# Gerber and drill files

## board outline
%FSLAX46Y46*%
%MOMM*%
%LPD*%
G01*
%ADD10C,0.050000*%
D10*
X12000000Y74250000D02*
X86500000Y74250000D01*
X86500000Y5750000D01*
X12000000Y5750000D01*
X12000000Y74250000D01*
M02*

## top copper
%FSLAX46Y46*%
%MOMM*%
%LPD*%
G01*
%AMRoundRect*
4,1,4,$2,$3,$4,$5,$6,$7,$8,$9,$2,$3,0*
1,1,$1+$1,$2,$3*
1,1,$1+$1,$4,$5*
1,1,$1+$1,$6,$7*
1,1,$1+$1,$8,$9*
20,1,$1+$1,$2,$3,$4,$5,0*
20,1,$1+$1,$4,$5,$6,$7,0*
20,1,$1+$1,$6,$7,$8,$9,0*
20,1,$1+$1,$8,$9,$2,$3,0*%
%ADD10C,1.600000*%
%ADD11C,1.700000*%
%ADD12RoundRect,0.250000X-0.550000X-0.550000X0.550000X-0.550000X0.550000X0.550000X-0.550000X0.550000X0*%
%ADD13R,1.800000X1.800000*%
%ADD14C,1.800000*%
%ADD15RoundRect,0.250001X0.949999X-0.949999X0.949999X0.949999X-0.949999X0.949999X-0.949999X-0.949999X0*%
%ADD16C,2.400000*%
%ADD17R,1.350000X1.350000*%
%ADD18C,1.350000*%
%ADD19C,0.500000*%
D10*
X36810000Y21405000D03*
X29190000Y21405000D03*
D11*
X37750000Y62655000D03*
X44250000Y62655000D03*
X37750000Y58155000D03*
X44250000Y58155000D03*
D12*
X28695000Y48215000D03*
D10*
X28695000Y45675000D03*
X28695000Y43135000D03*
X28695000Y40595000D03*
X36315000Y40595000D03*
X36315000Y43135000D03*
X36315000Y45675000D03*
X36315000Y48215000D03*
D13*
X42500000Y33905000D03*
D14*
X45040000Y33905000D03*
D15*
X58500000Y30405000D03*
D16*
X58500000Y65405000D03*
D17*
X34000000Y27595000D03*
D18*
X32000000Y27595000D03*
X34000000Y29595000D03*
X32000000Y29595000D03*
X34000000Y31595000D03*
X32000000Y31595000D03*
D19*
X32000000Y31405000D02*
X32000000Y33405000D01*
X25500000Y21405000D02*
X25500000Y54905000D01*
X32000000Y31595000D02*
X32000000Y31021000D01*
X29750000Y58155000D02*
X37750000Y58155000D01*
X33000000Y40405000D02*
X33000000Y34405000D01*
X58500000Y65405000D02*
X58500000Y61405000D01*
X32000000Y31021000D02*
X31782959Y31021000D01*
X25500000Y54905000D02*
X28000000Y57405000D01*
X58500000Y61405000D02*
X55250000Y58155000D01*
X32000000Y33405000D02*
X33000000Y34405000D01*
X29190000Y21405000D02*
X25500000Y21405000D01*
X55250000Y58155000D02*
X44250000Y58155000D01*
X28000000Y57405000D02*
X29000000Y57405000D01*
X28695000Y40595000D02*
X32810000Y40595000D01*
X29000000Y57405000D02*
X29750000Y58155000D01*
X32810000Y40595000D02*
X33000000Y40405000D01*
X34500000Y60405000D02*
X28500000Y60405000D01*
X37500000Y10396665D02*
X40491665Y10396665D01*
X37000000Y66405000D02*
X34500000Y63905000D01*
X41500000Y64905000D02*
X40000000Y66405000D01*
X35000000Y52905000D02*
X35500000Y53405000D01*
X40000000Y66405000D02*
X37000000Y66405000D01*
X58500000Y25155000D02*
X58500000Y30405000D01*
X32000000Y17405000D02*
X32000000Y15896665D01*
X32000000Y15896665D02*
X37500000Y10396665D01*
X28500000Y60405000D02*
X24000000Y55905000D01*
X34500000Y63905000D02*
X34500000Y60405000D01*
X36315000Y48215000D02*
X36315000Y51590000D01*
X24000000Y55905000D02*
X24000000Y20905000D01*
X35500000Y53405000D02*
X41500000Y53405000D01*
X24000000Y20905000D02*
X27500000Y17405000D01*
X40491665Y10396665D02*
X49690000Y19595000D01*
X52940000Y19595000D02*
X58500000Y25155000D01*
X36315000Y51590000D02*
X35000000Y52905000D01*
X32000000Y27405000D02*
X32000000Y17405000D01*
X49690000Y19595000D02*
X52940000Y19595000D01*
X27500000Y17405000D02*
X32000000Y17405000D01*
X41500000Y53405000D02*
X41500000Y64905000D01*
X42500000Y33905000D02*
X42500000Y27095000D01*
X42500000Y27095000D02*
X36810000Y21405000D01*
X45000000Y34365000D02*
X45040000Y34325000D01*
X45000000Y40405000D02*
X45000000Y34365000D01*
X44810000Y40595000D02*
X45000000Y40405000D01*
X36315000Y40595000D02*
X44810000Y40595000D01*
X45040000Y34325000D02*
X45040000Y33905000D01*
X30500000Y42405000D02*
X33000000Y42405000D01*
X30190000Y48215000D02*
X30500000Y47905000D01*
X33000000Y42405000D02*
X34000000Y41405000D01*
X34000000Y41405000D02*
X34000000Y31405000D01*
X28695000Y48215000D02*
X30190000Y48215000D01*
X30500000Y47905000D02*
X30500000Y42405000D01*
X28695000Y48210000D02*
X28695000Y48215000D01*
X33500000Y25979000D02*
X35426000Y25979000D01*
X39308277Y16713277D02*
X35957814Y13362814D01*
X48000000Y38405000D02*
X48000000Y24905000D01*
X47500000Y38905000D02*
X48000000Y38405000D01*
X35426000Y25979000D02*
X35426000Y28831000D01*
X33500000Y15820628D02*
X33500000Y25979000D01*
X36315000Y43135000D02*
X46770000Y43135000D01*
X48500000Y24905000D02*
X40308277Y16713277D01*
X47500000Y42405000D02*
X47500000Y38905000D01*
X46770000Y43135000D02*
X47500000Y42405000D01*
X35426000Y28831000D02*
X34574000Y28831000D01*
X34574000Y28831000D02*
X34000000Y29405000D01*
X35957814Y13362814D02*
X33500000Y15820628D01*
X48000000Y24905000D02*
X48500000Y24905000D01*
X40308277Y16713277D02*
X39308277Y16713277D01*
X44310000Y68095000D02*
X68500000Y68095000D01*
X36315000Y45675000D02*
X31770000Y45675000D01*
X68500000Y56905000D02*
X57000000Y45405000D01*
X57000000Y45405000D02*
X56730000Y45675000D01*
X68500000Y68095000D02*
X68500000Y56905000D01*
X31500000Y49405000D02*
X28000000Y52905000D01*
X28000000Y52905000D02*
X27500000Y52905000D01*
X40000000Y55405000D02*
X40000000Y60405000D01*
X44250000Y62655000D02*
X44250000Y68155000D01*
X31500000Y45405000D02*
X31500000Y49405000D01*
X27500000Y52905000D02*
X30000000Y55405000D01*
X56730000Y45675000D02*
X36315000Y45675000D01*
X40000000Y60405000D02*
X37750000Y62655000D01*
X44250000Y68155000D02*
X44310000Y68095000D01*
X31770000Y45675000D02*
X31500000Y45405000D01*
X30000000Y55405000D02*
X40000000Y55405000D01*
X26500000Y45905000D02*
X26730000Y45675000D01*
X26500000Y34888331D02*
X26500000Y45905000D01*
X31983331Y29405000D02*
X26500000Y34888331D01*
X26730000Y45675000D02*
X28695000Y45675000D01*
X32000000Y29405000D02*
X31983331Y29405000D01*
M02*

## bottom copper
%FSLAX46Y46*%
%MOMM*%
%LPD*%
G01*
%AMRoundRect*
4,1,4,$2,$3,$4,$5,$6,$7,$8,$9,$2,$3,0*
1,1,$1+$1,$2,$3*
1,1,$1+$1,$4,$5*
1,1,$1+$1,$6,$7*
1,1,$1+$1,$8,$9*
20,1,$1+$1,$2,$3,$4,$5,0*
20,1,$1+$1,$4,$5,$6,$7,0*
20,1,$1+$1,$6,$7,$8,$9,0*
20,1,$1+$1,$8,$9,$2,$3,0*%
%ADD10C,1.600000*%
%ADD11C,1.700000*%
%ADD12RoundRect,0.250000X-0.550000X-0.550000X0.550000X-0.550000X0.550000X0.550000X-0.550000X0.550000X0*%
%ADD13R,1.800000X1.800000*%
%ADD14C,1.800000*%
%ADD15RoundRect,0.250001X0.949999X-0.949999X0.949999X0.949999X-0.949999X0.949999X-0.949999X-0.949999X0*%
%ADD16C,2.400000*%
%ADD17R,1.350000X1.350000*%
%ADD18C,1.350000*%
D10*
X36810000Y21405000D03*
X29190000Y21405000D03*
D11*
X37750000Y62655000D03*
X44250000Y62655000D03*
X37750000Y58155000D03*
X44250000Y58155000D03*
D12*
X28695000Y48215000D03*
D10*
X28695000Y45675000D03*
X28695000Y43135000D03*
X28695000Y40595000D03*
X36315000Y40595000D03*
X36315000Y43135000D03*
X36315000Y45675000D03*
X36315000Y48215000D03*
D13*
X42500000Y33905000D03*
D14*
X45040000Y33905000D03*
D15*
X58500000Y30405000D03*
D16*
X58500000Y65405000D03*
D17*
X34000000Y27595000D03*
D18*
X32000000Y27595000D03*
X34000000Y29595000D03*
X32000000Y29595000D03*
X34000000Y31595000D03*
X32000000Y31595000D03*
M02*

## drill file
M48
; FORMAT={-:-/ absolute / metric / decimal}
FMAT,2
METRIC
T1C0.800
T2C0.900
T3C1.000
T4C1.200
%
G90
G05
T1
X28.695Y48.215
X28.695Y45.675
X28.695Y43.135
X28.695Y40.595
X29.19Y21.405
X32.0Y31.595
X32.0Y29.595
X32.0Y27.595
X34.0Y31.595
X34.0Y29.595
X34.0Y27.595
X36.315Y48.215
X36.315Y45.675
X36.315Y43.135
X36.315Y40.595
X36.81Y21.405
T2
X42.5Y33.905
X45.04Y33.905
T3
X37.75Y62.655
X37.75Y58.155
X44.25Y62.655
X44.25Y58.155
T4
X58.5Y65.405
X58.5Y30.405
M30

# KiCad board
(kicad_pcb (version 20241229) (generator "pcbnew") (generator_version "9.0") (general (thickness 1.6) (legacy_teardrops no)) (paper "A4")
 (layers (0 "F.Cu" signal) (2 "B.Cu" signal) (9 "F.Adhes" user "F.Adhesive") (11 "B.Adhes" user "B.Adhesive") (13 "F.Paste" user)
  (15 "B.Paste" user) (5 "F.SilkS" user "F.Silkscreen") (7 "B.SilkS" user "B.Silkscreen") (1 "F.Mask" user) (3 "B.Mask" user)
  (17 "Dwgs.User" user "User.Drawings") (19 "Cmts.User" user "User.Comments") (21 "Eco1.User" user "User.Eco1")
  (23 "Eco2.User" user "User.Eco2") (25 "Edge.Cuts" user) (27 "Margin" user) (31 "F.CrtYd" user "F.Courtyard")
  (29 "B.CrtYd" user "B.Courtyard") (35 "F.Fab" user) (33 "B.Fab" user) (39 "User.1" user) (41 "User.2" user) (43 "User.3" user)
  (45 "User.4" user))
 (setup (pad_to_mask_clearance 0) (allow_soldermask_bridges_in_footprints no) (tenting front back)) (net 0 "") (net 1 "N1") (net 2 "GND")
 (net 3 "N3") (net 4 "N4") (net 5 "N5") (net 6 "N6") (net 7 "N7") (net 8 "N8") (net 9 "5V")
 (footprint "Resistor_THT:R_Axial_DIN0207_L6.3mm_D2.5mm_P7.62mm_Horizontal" (layer "F.Cu") (at 36.81 -21.405 180)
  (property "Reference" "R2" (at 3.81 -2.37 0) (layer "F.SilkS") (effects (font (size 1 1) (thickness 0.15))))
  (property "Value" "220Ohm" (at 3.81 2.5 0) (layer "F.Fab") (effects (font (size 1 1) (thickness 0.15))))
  (pad "1" thru_hole circle (at 0 0 180) (size 1.6 1.6) (drill 0.8) (layers "*.Cu" "*.Mask") (remove_unused_layers no) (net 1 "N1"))
  (pad "2" thru_hole circle (at 7.62 0 180) (size 1.6 1.6) (drill 0.8) (layers "*.Cu" "*.Mask") (remove_unused_layers no) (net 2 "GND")))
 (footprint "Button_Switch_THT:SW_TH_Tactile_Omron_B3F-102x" (layer "F.Cu") (at 37.75 -62.655)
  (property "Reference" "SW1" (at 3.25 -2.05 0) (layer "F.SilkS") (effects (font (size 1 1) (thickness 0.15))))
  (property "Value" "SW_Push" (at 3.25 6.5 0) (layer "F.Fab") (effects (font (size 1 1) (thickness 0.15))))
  (pad "1" thru_hole circle (at 0 0) (size 1.7 1.7) (drill 1) (layers "*.Cu" "*.Mask") (remove_unused_layers no) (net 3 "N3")
   (thermal_bridge_angle 90))
  (pad "1" thru_hole circle (at 6.5 0) (size 1.7 1.7) (drill 1) (layers "*.Cu" "*.Mask") (remove_unused_layers no) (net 3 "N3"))
  (pad "2" thru_hole circle (at 0 4.5) (size 1.7 1.7) (drill 1) (layers "*.Cu" "*.Mask") (remove_unused_layers no) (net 2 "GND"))
  (pad "2" thru_hole circle (at 6.5 4.5) (size 1.7 1.7) (drill 1) (layers "*.Cu" "*.Mask") (remove_unused_layers no) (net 2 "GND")))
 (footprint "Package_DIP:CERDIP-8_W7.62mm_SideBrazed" (layer "F.Cu") (at 28.695 -48.215)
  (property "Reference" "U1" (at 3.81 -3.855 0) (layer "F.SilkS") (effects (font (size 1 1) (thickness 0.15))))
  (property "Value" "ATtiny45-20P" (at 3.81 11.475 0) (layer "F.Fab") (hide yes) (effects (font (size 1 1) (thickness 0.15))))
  (pad "1" thru_hole roundrect (at 0 0) (size 1.6 1.6) (drill 0.8) (layers "*.Cu" "*.Mask") (remove_unused_layers no)
   (roundrect_rratio 0.15625) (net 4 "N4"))
  (pad "2" thru_hole circle (at 0 2.54) (size 1.6 1.6) (drill 0.8) (layers "*.Cu" "*.Mask") (remove_unused_layers no) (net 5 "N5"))
  (pad "3" thru_hole circle (at 0 5.08) (size 1.6 1.6) (drill 0.8) (layers "*.Cu" "*.Mask") (remove_unused_layers no) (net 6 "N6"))
  (pad "4" thru_hole circle (at 0 7.62) (size 1.6 1.6) (drill 0.8) (layers "*.Cu" "*.Mask") (remove_unused_layers no) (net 2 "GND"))
  (pad "5" thru_hole circle (at 7.62 7.62) (size 1.6 1.6) (drill 0.8) (layers "*.Cu" "*.Mask") (remove_unused_layers no) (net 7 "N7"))
  (pad "6" thru_hole circle (at 7.62 5.08) (size 1.6 1.6) (drill 0.8) (layers "*.Cu" "*.Mask") (remove_unused_layers no) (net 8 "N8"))
  (pad "7" thru_hole circle (at 7.62 2.54) (size 1.6 1.6) (drill 0.8) (layers "*.Cu" "*.Mask") (remove_unused_layers no) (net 3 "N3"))
  (pad "8" thru_hole circle (at 7.62 0) (size 1.6 1.6) (drill 0.8) (layers "*.Cu" "*.Mask") (remove_unused_layers no) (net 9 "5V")))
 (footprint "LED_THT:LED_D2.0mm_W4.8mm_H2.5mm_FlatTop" (layer "F.Cu") (at 42.5 -33.905)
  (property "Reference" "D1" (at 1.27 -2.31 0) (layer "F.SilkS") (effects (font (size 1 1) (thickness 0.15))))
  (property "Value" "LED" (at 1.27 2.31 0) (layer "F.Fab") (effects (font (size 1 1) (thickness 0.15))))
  (pad "1" thru_hole rect (at 0 0) (size 1.8 1.8) (drill 0.9) (layers "*.Cu" "*.Mask") (remove_unused_layers no) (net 1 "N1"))
  (pad "2" thru_hole circle (at 2.54 0) (size 1.8 1.8) (drill 0.9) (layers "*.Cu" "*.Mask") (remove_unused_layers no) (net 7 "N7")))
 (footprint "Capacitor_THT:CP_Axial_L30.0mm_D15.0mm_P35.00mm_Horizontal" (layer "F.Cu") (at 58.5 -30.405 90)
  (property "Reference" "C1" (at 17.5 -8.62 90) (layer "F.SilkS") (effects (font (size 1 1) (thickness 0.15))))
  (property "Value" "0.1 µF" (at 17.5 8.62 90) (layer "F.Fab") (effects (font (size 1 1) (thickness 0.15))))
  (pad "1" thru_hole roundrect (at 0 0 90) (size 2.4 2.4) (drill 1.2) (layers "*.Cu" "*.Mask") (remove_unused_layers no)
   (roundrect_rratio 0.104167) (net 9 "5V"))
  (pad "2" thru_hole circle (at 35 0 90) (size 2.4 2.4) (drill 1.2) (layers "*.Cu" "*.Mask") (remove_unused_layers no) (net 2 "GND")))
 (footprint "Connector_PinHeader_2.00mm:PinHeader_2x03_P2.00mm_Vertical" (layer "F.Cu") (at 34 -27.595 180)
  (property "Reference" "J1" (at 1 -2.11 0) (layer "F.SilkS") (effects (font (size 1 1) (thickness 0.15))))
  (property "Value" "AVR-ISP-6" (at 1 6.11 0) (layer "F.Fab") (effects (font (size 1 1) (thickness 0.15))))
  (pad "0" thru_hole rect (at 0 0 180) (size 1.35 1.35) (drill 0.8) (layers "*.Cu" "*.Mask") (remove_unused_layers no) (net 6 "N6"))
  (pad "2" thru_hole circle (at 2 0 180) (size 1.35 1.35) (drill 0.8) (layers "*.Cu" "*.Mask") (remove_unused_layers no) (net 9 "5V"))
  (pad "3" thru_hole circle (at 0 2 180) (size 1.35 1.35) (drill 0.8) (layers "*.Cu" "*.Mask") (remove_unused_layers no) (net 8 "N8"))
  (pad "4" thru_hole circle (at 2 2 180) (size 1.35 1.35) (drill 0.8) (layers "*.Cu" "*.Mask") (remove_unused_layers no) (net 5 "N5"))
  (pad "5" thru_hole circle (at 0 4 180) (size 1.35 1.35) (drill 0.8) (layers "*.Cu" "*.Mask") (remove_unused_layers no) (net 4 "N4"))
  (pad "6" thru_hole circle (at 2 4 180) (size 1.35 1.35) (drill 0.8) (layers "*.Cu" "*.Mask") (remove_unused_layers no) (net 2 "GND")))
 (gr_rect (start 12 -74.25) (end 86.5 -5.75) (stroke (width 0.05) (type default)) (fill no) (layer "Edge.Cuts"))
 (segment (start 32 -31.405) (end 32 -33.405) (width 0.5) (layer "F.Cu") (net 2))
 (segment (start 25.5 -21.405) (end 25.5 -54.905) (width 0.5) (layer "F.Cu") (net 2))
 (segment (start 32 -31.595) (end 32 -31.021) (width 0.5) (layer "F.Cu") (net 2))
 (segment (start 29.75 -58.155) (end 37.75 -58.155) (width 0.5) (layer "F.Cu") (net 2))
 (segment (start 33 -40.405) (end 33 -34.405) (width 0.5) (layer "F.Cu") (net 2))
 (segment (start 58.5 -65.405) (end 58.5 -61.405) (width 0.5) (layer "F.Cu") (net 2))
 (segment (start 32 -31.021) (end 31.782959 -31.021) (width 0.5) (layer "F.Cu") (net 2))
 (segment (start 25.5 -54.905) (end 28 -57.405) (width 0.5) (layer "F.Cu") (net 2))
 (segment (start 58.5 -61.405) (end 55.25 -58.155) (width 0.5) (layer "F.Cu") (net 2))
 (segment (start 32 -33.405) (end 33 -34.405) (width 0.5) (layer "F.Cu") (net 2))
 (segment (start 29.19 -21.405) (end 25.5 -21.405) (width 0.5) (layer "F.Cu") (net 2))
 (segment (start 55.25 -58.155) (end 44.25 -58.155) (width 0.5) (layer "F.Cu") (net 2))
 (segment (start 28 -57.405) (end 29 -57.405) (width 0.5) (layer "F.Cu") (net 2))
 (segment (start 28.695 -40.595) (end 32.81 -40.595) (width 0.5) (layer "F.Cu") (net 2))
 (segment (start 29 -57.405) (end 29.75 -58.155) (width 0.5) (layer "F.Cu") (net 2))
 (segment (start 32.81 -40.595) (end 33 -40.405) (width 0.5) (layer "F.Cu") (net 2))
 (segment (start 34.5 -60.405) (end 28.5 -60.405) (width 0.5) (layer "F.Cu") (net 9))
 (segment (start 37.5 -10.396665) (end 40.491665 -10.396665) (width 0.5) (layer "F.Cu") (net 9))
 (segment (start 37 -66.405) (end 34.5 -63.905) (width 0.5) (layer "F.Cu") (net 9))
 (segment (start 41.5 -64.905) (end 40 -66.405) (width 0.5) (layer "F.Cu") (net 9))
 (segment (start 35 -52.905) (end 35.5 -53.405) (width 0.5) (layer "F.Cu") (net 9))
 (segment (start 40 -66.405) (end 37 -66.405) (width 0.5) (layer "F.Cu") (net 9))
 (segment (start 58.5 -25.155) (end 58.5 -30.405) (width 0.5) (layer "F.Cu") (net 9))
 (segment (start 32 -17.405) (end 32 -15.896665) (width 0.5) (layer "F.Cu") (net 9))
 (segment (start 32 -15.896665) (end 37.5 -10.396665) (width 0.5) (layer "F.Cu") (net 9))
 (segment (start 28.5 -60.405) (end 24 -55.905) (width 0.5) (layer "F.Cu") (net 9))
 (segment (start 34.5 -63.905) (end 34.5 -60.405) (width 0.5) (layer "F.Cu") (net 9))
 (segment (start 36.315 -48.215) (end 36.315 -51.59) (width 0.5) (layer "F.Cu") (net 9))
 (segment (start 24 -55.905) (end 24 -20.905) (width 0.5) (layer "F.Cu") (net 9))
 (segment (start 35.5 -53.405) (end 41.5 -53.405) (width 0.5) (layer "F.Cu") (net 9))
 (segment (start 24 -20.905) (end 27.5 -17.405) (width 0.5) (layer "F.Cu") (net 9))
 (segment (start 40.491665 -10.396665) (end 49.69 -19.595) (width 0.5) (layer "F.Cu") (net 9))
 (segment (start 52.94 -19.595) (end 58.5 -25.155) (width 0.5) (layer "F.Cu") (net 9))
 (segment (start 36.315 -51.59) (end 35 -52.905) (width 0.5) (layer "F.Cu") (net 9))
 (segment (start 32 -27.405) (end 32 -17.405) (width 0.5) (layer "F.Cu") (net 9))
 (segment (start 49.69 -19.595) (end 52.94 -19.595) (width 0.5) (layer "F.Cu") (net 9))
 (segment (start 27.5 -17.405) (end 32 -17.405) (width 0.5) (layer "F.Cu") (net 9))
 (segment (start 41.5 -53.405) (end 41.5 -64.905) (width 0.5) (layer "F.Cu") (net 9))
 (segment (start 42.5 -33.905) (end 42.5 -27.095) (width 0.5) (layer "F.Cu") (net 1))
 (segment (start 42.5 -27.095) (end 36.81 -21.405) (width 0.5) (layer "F.Cu") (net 1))
 (segment (start 45 -34.365) (end 45.04 -34.325) (width 0.5) (layer "F.Cu") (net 7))
 (segment (start 45 -40.405) (end 45 -34.365) (width 0.5) (layer "F.Cu") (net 7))
 (segment (start 44.81 -40.595) (end 45 -40.405) (width 0.5) (layer "F.Cu") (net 7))
 (segment (start 36.315 -40.595) (end 44.81 -40.595) (width 0.5) (layer "F.Cu") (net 7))
 (segment (start 45.04 -34.325) (end 45.04 -33.905) (width 0.5) (layer "F.Cu") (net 7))
 (segment (start 30.5 -42.405) (end 33 -42.405) (width 0.5) (layer "F.Cu") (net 4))
 (segment (start 30.19 -48.215) (end 30.5 -47.905) (width 0.5) (layer "F.Cu") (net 4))
 (segment (start 33 -42.405) (end 34 -41.405) (width 0.5) (layer "F.Cu") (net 4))
 (segment (start 34 -41.405) (end 34 -31.405) (width 0.5) (layer "F.Cu") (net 4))
 (segment (start 28.695 -48.215) (end 30.19 -48.215) (width 0.5) (layer "F.Cu") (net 4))
 (segment (start 30.5 -47.905) (end 30.5 -42.405) (width 0.5) (layer "F.Cu") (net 4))
 (segment (start 28.695 -48.21) (end 28.695 -48.215) (width 0.5) (layer "F.Cu") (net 4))
 (segment (start 33.5 -25.979) (end 35.426 -25.979) (width 0.5) (layer "F.Cu") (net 8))
 (segment (start 39.308277 -16.713277) (end 35.957814 -13.362814) (width 0.5) (layer "F.Cu") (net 8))
 (segment (start 48 -38.405) (end 48 -24.905) (width 0.5) (layer "F.Cu") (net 8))
 (segment (start 47.5 -38.905) (end 48 -38.405) (width 0.5) (layer "F.Cu") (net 8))
 (segment (start 35.426 -25.979) (end 35.426 -28.831) (width 0.5) (layer "F.Cu") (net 8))
 (segment (start 33.5 -15.820628) (end 33.5 -25.979) (width 0.5) (layer "F.Cu") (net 8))
 (segment (start 36.315 -43.135) (end 46.77 -43.135) (width 0.5) (layer "F.Cu") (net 8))
 (segment (start 48.5 -24.905) (end 40.308277 -16.713277) (width 0.5) (layer "F.Cu") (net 8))
 (segment (start 47.5 -42.405) (end 47.5 -38.905) (width 0.5) (layer "F.Cu") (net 8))
 (segment (start 46.77 -43.135) (end 47.5 -42.405) (width 0.5) (layer "F.Cu") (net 8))
 (segment (start 35.426 -28.831) (end 34.574 -28.831) (width 0.5) (layer "F.Cu") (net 8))
 (segment (start 34.574 -28.831) (end 34 -29.405) (width 0.5) (layer "F.Cu") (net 8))
 (segment (start 35.957814 -13.362814) (end 33.5 -15.820628) (width 0.5) (layer "F.Cu") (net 8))
 (segment (start 48 -24.905) (end 48.5 -24.905) (width 0.5) (layer "F.Cu") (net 8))
 (segment (start 40.308277 -16.713277) (end 39.308277 -16.713277) (width 0.5) (layer "F.Cu") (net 8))
 (segment (start 44.31 -68.095) (end 68.5 -68.095) (width 0.5) (layer "F.Cu") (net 3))
 (segment (start 36.315 -45.675) (end 31.77 -45.675) (width 0.5) (layer "F.Cu") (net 3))
 (segment (start 68.5 -56.905) (end 57 -45.405) (width 0.5) (layer "F.Cu") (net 3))
 (segment (start 57 -45.405) (end 56.73 -45.675) (width 0.5) (layer "F.Cu") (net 3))
 (segment (start 68.5 -68.095) (end 68.5 -56.905) (width 0.5) (layer "F.Cu") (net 3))
 (segment (start 31.5 -49.405) (end 28 -52.905) (width 0.5) (layer "F.Cu") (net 3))
 (segment (start 28 -52.905) (end 27.5 -52.905) (width 0.5) (layer "F.Cu") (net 3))
 (segment (start 40 -55.405) (end 40 -60.405) (width 0.5) (layer "F.Cu") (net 3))
 (segment (start 44.25 -62.655) (end 44.25 -68.155) (width 0.5) (layer "F.Cu") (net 3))
 (segment (start 31.5 -45.405) (end 31.5 -49.405) (width 0.5) (layer "F.Cu") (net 3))
 (segment (start 27.5 -52.905) (end 30 -55.405) (width 0.5) (layer "F.Cu") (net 3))
 (segment (start 56.73 -45.675) (end 36.315 -45.675) (width 0.5) (layer "F.Cu") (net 3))
 (segment (start 40 -60.405) (end 37.75 -62.655) (width 0.5) (layer "F.Cu") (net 3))
 (segment (start 44.25 -68.155) (end 44.31 -68.095) (width 0.5) (layer "F.Cu") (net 3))
 (segment (start 31.77 -45.675) (end 31.5 -45.405) (width 0.5) (layer "F.Cu") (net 3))
 (segment (start 30 -55.405) (end 40 -55.405) (width 0.5) (layer "F.Cu") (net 3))
 (segment (start 26.5 -45.905) (end 26.73 -45.675) (width 0.5) (layer "F.Cu") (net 5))
 (segment (start 26.5 -34.888331) (end 26.5 -45.905) (width 0.5) (layer "F.Cu") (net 5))
 (segment (start 31.983331 -29.405) (end 26.5 -34.888331) (width 0.5) (layer "F.Cu") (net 5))
 (segment (start 26.73 -45.675) (end 28.695 -45.675) (width 0.5) (layer "F.Cu") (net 5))
 (segment (start 32 -29.405) (end 31.983331 -29.405) (width 0.5) (layer "F.Cu") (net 5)))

